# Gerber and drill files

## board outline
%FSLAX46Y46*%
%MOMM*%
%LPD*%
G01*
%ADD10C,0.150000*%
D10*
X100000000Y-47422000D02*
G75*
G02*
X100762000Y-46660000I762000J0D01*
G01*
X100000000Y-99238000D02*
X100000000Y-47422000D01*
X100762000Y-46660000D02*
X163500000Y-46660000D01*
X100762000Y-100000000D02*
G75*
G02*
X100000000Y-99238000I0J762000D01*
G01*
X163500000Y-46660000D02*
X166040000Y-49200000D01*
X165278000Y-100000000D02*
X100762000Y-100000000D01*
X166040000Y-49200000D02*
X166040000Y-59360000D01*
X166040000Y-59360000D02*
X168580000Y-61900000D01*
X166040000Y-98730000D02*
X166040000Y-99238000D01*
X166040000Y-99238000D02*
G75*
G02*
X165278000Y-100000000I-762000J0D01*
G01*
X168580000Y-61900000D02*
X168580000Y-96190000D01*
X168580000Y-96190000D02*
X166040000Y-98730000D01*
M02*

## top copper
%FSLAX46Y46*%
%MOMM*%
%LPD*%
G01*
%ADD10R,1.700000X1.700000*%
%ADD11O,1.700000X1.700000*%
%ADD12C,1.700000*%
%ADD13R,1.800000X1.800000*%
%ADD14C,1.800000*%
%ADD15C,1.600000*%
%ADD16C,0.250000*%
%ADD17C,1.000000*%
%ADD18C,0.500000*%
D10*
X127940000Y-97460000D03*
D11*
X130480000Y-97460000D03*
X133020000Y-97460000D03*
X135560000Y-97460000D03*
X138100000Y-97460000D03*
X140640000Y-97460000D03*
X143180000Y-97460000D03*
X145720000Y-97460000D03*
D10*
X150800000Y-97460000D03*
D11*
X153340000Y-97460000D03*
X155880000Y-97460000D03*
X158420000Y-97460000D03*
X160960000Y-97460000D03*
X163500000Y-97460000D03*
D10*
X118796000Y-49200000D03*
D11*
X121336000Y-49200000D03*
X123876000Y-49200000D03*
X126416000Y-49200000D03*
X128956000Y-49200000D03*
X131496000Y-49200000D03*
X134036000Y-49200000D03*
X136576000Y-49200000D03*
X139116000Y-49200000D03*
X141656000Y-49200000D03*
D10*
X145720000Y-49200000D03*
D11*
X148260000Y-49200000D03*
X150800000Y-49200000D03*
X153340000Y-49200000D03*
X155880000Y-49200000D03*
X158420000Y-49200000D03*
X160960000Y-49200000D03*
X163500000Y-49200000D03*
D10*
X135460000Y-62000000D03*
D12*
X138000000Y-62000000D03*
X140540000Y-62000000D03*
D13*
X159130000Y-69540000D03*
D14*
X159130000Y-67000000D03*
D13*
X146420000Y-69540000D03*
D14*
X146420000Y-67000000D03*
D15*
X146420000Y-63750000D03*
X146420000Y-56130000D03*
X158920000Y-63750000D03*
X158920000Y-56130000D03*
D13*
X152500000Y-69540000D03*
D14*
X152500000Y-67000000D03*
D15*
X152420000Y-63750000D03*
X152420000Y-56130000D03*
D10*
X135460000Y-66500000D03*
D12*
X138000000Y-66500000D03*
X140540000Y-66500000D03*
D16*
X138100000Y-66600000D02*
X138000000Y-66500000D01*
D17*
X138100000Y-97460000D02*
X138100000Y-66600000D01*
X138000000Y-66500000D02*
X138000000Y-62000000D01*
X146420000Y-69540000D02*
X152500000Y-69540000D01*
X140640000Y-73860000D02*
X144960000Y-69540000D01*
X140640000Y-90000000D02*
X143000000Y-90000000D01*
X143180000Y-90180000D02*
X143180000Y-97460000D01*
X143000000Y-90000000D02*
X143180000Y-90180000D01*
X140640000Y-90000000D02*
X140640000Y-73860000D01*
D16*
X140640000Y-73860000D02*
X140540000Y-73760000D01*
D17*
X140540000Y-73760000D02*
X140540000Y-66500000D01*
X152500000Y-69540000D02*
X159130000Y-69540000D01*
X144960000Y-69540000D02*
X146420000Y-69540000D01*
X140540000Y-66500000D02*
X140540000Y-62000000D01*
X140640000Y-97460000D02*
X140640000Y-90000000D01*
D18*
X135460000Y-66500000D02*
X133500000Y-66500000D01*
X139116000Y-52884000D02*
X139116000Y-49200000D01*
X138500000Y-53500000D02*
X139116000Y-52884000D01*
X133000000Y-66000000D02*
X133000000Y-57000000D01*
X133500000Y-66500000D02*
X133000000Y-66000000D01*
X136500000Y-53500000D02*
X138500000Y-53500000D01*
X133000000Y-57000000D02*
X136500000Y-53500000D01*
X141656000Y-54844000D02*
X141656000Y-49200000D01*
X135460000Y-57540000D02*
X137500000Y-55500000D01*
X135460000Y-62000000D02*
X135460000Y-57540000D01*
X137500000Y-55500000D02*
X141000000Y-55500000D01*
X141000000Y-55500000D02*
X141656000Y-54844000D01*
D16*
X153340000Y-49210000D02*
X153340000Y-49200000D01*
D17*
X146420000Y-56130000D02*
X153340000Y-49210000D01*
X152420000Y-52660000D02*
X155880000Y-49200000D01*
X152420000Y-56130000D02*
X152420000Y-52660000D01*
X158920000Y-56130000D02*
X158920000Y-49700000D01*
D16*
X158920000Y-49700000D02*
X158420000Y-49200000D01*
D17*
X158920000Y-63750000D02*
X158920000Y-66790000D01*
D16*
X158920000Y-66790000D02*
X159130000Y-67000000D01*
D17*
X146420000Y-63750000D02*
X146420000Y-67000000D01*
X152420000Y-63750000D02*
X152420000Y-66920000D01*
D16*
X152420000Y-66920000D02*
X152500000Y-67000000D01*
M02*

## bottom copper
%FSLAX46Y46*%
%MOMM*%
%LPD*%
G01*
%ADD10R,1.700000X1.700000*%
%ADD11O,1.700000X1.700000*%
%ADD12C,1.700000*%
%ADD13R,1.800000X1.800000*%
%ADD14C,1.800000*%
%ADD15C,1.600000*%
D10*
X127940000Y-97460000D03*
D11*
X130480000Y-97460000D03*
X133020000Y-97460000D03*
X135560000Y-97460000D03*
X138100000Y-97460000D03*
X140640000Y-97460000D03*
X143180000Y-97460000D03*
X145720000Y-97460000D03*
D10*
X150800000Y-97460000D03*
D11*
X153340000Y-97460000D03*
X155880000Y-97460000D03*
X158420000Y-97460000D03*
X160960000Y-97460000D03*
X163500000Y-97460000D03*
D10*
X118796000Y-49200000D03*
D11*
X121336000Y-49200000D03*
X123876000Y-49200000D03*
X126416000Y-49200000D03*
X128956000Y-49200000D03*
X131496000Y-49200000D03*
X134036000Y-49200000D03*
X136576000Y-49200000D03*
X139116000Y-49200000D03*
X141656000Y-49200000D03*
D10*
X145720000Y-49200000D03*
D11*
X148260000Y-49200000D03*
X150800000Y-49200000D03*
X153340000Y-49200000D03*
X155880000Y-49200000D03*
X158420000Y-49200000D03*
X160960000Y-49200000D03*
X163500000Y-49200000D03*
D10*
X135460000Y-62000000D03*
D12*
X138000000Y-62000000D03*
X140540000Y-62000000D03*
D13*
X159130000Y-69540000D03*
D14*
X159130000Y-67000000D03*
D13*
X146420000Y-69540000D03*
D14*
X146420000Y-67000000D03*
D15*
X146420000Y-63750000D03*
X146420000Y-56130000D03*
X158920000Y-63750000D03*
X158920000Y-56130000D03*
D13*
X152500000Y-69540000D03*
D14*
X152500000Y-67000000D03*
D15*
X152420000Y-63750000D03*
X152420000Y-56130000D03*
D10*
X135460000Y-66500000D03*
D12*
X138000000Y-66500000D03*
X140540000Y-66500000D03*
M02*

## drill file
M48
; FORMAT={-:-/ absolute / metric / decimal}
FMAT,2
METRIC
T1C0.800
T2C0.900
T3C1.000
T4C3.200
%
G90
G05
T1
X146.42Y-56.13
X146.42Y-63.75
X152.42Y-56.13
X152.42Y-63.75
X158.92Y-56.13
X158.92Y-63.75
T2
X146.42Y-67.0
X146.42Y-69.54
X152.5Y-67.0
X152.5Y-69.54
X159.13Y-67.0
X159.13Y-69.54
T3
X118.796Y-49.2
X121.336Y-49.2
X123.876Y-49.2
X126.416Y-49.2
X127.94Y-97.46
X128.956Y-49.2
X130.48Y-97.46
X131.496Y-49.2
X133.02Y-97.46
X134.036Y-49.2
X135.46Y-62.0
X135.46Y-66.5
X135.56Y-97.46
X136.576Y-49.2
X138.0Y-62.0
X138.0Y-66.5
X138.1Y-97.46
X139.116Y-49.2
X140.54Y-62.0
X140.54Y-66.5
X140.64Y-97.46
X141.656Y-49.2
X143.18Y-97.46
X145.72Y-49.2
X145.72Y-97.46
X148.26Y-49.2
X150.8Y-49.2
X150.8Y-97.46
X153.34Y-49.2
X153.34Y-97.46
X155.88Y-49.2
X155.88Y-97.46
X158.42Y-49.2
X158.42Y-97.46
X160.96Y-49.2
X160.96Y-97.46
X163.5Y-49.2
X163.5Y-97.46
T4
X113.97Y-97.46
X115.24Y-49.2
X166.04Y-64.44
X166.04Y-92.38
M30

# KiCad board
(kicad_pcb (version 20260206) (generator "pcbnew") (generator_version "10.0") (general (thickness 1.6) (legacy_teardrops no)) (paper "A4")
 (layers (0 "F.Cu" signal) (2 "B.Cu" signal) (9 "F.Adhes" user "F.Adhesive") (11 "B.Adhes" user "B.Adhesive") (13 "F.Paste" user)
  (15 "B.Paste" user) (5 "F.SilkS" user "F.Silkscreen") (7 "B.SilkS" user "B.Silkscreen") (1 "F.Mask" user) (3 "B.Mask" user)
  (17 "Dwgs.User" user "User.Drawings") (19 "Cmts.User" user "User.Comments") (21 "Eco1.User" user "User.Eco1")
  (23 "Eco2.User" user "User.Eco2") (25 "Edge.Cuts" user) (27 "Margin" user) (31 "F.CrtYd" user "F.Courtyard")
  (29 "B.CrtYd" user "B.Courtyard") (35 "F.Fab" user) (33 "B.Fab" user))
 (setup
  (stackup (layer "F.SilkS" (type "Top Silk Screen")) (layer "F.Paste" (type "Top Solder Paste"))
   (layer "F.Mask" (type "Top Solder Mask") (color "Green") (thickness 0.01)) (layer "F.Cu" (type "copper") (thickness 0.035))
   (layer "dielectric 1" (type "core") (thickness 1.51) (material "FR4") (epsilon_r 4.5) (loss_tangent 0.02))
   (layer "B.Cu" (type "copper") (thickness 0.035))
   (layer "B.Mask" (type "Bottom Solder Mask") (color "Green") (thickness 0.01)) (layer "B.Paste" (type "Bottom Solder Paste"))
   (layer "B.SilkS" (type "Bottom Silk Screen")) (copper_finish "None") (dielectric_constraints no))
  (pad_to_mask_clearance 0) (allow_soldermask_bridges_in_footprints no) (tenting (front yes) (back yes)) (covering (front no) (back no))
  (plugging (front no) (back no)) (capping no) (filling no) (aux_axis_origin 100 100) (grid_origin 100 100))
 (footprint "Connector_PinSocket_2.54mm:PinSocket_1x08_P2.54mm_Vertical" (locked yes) (layer "F.Cu") (at 127.94 97.46 90)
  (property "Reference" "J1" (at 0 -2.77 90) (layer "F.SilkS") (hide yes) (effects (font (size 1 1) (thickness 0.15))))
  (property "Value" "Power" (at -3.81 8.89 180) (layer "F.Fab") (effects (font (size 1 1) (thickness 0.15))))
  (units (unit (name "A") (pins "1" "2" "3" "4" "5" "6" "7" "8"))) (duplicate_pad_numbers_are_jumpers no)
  (pad "1" thru_hole rect (at 0 0 90) (size 1.7 1.7) (drill 1) (layers "*.Cu" "*.Mask") (remove_unused_layers no)
   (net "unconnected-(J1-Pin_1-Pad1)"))
  (pad "2" thru_hole oval (at 0 2.54 90) (size 1.7 1.7) (drill 1) (layers "*.Cu" "*.Mask") (remove_unused_layers no)
   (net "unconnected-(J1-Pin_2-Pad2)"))
  (pad "3" thru_hole oval (at 0 5.08 90) (size 1.7 1.7) (drill 1) (layers "*.Cu" "*.Mask") (remove_unused_layers no)
   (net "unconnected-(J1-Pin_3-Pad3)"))
  (pad "4" thru_hole oval (at 0 7.62 90) (size 1.7 1.7) (drill 1) (layers "*.Cu" "*.Mask") (remove_unused_layers no) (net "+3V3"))
  (pad "5" thru_hole oval (at 0 10.16 90) (size 1.7 1.7) (drill 1) (layers "*.Cu" "*.Mask") (remove_unused_layers no) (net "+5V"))
  (pad "6" thru_hole oval (at 0 12.7 90) (size 1.7 1.7) (drill 1) (layers "*.Cu" "*.Mask") (remove_unused_layers no) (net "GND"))
  (pad "7" thru_hole oval (at 0 15.24 90) (size 1.7 1.7) (drill 1) (layers "*.Cu" "*.Mask") (remove_unused_layers no) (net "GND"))
  (pad "8" thru_hole oval (at 0 17.78 90) (size 1.7 1.7) (drill 1) (layers "*.Cu" "*.Mask") (remove_unused_layers no)
   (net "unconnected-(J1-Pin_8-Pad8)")))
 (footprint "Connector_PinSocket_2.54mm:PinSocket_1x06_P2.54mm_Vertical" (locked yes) (layer "F.Cu") (at 150.8 97.46 90)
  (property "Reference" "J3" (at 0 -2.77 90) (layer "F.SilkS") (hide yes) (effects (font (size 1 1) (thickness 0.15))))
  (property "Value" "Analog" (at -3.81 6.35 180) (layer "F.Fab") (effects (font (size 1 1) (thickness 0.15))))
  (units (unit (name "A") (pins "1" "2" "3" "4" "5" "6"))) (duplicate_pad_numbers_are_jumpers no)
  (pad "1" thru_hole rect (at 0 0 90) (size 1.7 1.7) (drill 1) (layers "*.Cu" "*.Mask") (remove_unused_layers no) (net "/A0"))
  (pad "2" thru_hole oval (at 0 2.54 90) (size 1.7 1.7) (drill 1) (layers "*.Cu" "*.Mask") (remove_unused_layers no) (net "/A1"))
  (pad "3" thru_hole oval (at 0 5.08 90) (size 1.7 1.7) (drill 1) (layers "*.Cu" "*.Mask") (remove_unused_layers no) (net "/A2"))
  (pad "4" thru_hole oval (at 0 7.62 90) (size 1.7 1.7) (drill 1) (layers "*.Cu" "*.Mask") (remove_unused_layers no) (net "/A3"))
  (pad "5" thru_hole oval (at 0 10.16 90) (size 1.7 1.7) (drill 1) (layers "*.Cu" "*.Mask") (remove_unused_layers no)
   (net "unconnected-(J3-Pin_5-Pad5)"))
  (pad "6" thru_hole oval (at 0 12.7 90) (size 1.7 1.7) (drill 1) (layers "*.Cu" "*.Mask") (remove_unused_layers no)
   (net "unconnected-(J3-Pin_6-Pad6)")))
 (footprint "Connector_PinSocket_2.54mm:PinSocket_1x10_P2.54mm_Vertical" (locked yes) (layer "F.Cu") (at 118.796 49.2 90)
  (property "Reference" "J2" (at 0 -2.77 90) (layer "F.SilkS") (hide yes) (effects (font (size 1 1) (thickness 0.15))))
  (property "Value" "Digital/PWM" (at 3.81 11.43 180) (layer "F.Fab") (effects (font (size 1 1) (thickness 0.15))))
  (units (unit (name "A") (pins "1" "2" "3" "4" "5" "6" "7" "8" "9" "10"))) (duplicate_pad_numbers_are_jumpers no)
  (pad "1" thru_hole rect (at 0 0 90) (size 1.7 1.7) (drill 1) (layers "*.Cu" "*.Mask") (remove_unused_layers no) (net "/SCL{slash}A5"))
  (pad "2" thru_hole oval (at 0 2.54 90) (size 1.7 1.7) (drill 1) (layers "*.Cu" "*.Mask") (remove_unused_layers no) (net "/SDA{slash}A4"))
  (pad "3" thru_hole oval (at 0 5.08 90) (size 1.7 1.7) (drill 1) (layers "*.Cu" "*.Mask") (remove_unused_layers no) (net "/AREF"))
  (pad "4" thru_hole oval (at 0 7.62 90) (size 1.7 1.7) (drill 1) (layers "*.Cu" "*.Mask") (remove_unused_layers no)
   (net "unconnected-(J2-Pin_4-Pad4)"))
  (pad "5" thru_hole oval (at 0 10.16 90) (size 1.7 1.7) (drill 1) (layers "*.Cu" "*.Mask") (remove_unused_layers no) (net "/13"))
  (pad "6" thru_hole oval (at 0 12.7 90) (size 1.7 1.7) (drill 1) (layers "*.Cu" "*.Mask") (remove_unused_layers no) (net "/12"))
  (pad "7" thru_hole oval (at 0 15.24 90) (size 1.7 1.7) (drill 1) (layers "*.Cu" "*.Mask") (remove_unused_layers no) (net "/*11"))
  (pad "8" thru_hole oval (at 0 17.78 90) (size 1.7 1.7) (drill 1) (layers "*.Cu" "*.Mask") (remove_unused_layers no) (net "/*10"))
  (pad "9" thru_hole oval (at 0 20.32 90) (size 1.7 1.7) (drill 1) (layers "*.Cu" "*.Mask") (remove_unused_layers no) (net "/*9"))
  (pad "10" thru_hole oval (at 0 22.86 90) (size 1.7 1.7) (drill 1) (layers "*.Cu" "*.Mask") (remove_unused_layers no) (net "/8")))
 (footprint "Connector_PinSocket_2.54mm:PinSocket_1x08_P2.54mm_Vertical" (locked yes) (layer "F.Cu") (at 145.72 49.2 90)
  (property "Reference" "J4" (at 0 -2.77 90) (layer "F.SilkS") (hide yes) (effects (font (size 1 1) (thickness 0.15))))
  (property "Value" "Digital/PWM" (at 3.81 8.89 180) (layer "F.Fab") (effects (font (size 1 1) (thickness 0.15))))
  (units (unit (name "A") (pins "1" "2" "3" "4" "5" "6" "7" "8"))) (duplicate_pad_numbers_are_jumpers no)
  (pad "1" thru_hole rect (at 0 0 90) (size 1.7 1.7) (drill 1) (layers "*.Cu" "*.Mask") (remove_unused_layers no) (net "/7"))
  (pad "2" thru_hole oval (at 0 2.54 90) (size 1.7 1.7) (drill 1) (layers "*.Cu" "*.Mask") (remove_unused_layers no) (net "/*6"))
  (pad "3" thru_hole oval (at 0 5.08 90) (size 1.7 1.7) (drill 1) (layers "*.Cu" "*.Mask") (remove_unused_layers no) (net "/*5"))
  (pad "4" thru_hole oval (at 0 7.62 90) (size 1.7 1.7) (drill 1) (layers "*.Cu" "*.Mask") (remove_unused_layers no) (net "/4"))
  (pad "5" thru_hole oval (at 0 10.16 90) (size 1.7 1.7) (drill 1) (layers "*.Cu" "*.Mask") (remove_unused_layers no) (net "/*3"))
  (pad "6" thru_hole oval (at 0 12.7 90) (size 1.7 1.7) (drill 1) (layers "*.Cu" "*.Mask") (remove_unused_layers no) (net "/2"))
  (pad "7" thru_hole oval (at 0 15.24 90) (size 1.7 1.7) (drill 1) (layers "*.Cu" "*.Mask") (remove_unused_layers no) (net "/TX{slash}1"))
  (pad "8" thru_hole oval (at 0 17.78 90) (size 1.7 1.7) (drill 1) (layers "*.Cu" "*.Mask") (remove_unused_layers no) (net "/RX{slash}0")))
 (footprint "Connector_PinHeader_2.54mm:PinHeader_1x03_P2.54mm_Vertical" (layer "F.Cu") (at 135.46 62 90)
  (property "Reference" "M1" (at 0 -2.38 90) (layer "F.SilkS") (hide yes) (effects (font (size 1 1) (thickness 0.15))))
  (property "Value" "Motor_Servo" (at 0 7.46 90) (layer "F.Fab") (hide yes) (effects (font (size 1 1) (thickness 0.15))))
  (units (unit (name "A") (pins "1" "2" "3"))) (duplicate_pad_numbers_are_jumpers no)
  (pad "1" thru_hole rect (at 0 0 90) (size 1.7 1.7) (drill 1) (layers "*.Cu" "*.Mask") (remove_unused_layers no) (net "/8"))
  (pad "2" thru_hole circle (at 0 2.54 90) (size 1.7 1.7) (drill 1) (layers "*.Cu" "*.Mask") (remove_unused_layers no) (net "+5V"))
  (pad "3" thru_hole circle (at 0 5.08 90) (size 1.7 1.7) (drill 1) (layers "*.Cu" "*.Mask") (remove_unused_layers no) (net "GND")))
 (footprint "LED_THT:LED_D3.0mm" (layer "F.Cu") (at 159.13 69.54 90)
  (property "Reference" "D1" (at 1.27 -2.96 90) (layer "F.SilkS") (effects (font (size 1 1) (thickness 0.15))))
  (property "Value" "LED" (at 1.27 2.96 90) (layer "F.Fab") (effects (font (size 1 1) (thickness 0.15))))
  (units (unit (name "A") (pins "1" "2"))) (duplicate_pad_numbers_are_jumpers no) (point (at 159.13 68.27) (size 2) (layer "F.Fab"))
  (pad "1" thru_hole rect (at 0 0 90) (size 1.8 1.8) (drill 0.9) (layers "*.Cu" "*.Mask") (remove_unused_layers no) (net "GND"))
  (pad "2" thru_hole circle (at 2.54 0 90) (size 1.8 1.8) (drill 0.9) (layers "*.Cu" "*.Mask") (remove_unused_layers no) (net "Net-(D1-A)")))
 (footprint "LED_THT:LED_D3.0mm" (layer "F.Cu") (at 146.42 69.54 90)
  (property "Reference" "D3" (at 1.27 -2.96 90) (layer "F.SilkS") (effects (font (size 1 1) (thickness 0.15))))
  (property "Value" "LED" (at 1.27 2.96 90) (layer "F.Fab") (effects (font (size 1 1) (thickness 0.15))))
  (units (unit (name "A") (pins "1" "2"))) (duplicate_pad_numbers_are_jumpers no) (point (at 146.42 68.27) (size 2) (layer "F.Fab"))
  (pad "1" thru_hole rect (at 0 0 90) (size 1.8 1.8) (drill 0.9) (layers "*.Cu" "*.Mask") (remove_unused_layers no) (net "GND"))
  (pad "2" thru_hole circle (at 2.54 0 90) (size 1.8 1.8) (drill 0.9) (layers "*.Cu" "*.Mask") (remove_unused_layers no) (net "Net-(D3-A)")))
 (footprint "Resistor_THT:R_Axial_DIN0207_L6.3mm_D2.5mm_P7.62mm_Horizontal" (layer "F.Cu") (at 146.42 63.75 90)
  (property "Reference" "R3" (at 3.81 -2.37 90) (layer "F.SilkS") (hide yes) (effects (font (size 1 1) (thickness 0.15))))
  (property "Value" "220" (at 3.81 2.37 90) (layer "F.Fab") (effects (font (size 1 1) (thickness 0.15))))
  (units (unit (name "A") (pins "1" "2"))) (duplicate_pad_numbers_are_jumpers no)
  (pad "1" thru_hole circle (at 0 0 90) (size 1.6 1.6) (drill 0.8) (layers "*.Cu" "*.Mask") (remove_unused_layers no) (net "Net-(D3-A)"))
  (pad "2" thru_hole circle (at 7.62 0 90) (size 1.6 1.6) (drill 0.8) (layers "*.Cu" "*.Mask") (remove_unused_layers no) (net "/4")))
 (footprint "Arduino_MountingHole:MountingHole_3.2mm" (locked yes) (layer "F.Cu") (at 115.24 49.2)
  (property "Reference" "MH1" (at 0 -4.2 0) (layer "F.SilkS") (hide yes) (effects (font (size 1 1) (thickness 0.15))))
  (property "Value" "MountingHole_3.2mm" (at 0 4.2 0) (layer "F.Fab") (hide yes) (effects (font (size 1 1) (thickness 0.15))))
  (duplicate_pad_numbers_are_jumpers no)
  (pad "" np_thru_hole circle (at 0 0) (size 3.2 3.2) (drill 3.2) (layers "*.Cu" "*.Mask")))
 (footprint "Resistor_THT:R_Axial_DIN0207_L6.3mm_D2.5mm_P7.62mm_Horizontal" (layer "F.Cu") (at 158.92 63.75 90)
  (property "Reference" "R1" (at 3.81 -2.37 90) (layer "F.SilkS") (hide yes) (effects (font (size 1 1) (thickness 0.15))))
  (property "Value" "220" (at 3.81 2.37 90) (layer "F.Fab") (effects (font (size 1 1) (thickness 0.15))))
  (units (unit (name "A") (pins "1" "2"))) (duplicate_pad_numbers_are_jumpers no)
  (pad "1" thru_hole circle (at 0 0 90) (size 1.6 1.6) (drill 0.8) (layers "*.Cu" "*.Mask") (remove_unused_layers no) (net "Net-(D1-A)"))
  (pad "2" thru_hole circle (at 7.62 0 90) (size 1.6 1.6) (drill 0.8) (layers "*.Cu" "*.Mask") (remove_unused_layers no) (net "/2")))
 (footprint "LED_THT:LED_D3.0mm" (layer "F.Cu") (at 152.5 69.54 90)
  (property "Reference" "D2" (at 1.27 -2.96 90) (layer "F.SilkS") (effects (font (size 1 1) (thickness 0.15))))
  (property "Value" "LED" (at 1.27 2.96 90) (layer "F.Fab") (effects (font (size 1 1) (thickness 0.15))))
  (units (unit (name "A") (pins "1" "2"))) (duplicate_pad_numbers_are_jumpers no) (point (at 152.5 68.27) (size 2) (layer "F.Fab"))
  (pad "1" thru_hole rect (at 0 0 90) (size 1.8 1.8) (drill 0.9) (layers "*.Cu" "*.Mask") (remove_unused_layers no) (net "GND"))
  (pad "2" thru_hole circle (at 2.54 0 90) (size 1.8 1.8) (drill 0.9) (layers "*.Cu" "*.Mask") (remove_unused_layers no) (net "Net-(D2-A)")))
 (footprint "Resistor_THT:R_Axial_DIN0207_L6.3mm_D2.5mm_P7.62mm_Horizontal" (layer "F.Cu") (at 152.42 63.75 90)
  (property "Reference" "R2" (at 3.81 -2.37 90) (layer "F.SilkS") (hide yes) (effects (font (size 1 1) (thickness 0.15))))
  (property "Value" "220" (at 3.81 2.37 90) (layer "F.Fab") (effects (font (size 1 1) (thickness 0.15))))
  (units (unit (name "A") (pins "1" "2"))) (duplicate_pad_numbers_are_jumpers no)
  (pad "1" thru_hole circle (at 0 0 90) (size 1.6 1.6) (drill 0.8) (layers "*.Cu" "*.Mask") (remove_unused_layers no) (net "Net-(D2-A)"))
  (pad "2" thru_hole circle (at 7.62 0 90) (size 1.6 1.6) (drill 0.8) (layers "*.Cu" "*.Mask") (remove_unused_layers no) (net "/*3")))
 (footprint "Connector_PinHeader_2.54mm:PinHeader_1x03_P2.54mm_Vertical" (layer "F.Cu") (at 135.46 66.5 90)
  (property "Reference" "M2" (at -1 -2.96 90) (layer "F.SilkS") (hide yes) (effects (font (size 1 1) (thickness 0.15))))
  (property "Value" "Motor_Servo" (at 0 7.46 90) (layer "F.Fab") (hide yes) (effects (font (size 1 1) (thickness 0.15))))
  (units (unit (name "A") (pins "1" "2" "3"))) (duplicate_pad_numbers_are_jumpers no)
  (pad "1" thru_hole rect (at 0 0 90) (size 1.7 1.7) (drill 1) (layers "*.Cu" "*.Mask") (remove_unused_layers no) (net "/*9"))
  (pad "2" thru_hole circle (at 0 2.54 90) (size 1.7 1.7) (drill 1) (layers "*.Cu" "*.Mask") (remove_unused_layers no) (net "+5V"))
  (pad "3" thru_hole circle (at 0 5.08 90) (size 1.7 1.7) (drill 1) (layers "*.Cu" "*.Mask") (remove_unused_layers no) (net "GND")))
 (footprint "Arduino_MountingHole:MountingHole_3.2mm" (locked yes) (layer "F.Cu") (at 113.97 97.46)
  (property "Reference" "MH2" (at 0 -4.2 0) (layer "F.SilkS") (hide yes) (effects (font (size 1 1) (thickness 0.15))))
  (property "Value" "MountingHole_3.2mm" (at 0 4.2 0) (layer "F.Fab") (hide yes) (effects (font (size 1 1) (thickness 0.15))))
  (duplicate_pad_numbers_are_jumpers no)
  (pad "" np_thru_hole circle (at 0 0) (size 3.2 3.2) (drill 3.2) (layers "*.Cu" "*.Mask")))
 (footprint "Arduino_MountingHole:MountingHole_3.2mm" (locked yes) (layer "F.Cu") (at 166.04 64.44)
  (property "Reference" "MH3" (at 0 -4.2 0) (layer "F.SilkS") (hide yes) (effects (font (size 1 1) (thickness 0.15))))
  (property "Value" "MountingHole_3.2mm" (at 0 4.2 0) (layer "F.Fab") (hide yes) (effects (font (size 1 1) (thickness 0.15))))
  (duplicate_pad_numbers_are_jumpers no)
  (pad "" np_thru_hole circle (at 0 0) (size 3.2 3.2) (drill 3.2) (layers "*.Cu" "*.Mask")))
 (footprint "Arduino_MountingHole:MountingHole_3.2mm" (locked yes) (layer "F.Cu") (at 166.04 92.38)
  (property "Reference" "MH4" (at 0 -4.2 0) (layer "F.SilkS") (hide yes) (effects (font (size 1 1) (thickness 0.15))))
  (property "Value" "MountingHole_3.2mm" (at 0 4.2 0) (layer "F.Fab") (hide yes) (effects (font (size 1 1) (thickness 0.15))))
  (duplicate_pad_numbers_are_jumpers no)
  (pad "" np_thru_hole circle (at 0 0) (size 3.2 3.2) (drill 3.2) (layers "*.Cu" "*.Mask")))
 (gr_arc (start 100 47.422) (mid 100.223185 46.883185) (end 100.762 46.66) (stroke (width 0.15) (type solid)) (layer "Edge.Cuts"))
 (gr_line (start 100 99.238) (end 100 47.422) (stroke (width 0.15) (type solid)) (layer "Edge.Cuts"))
 (gr_line (start 100.762 46.66) (end 163.5 46.66) (stroke (width 0.15) (type solid)) (layer "Edge.Cuts"))
 (gr_arc (start 100.762 100) (mid 100.223185 99.776815) (end 100 99.238) (stroke (width 0.15) (type solid)) (layer "Edge.Cuts"))
 (gr_line (start 163.5 46.66) (end 166.04 49.2) (stroke (width 0.15) (type solid)) (layer "Edge.Cuts"))
 (gr_line (start 165.278 100) (end 100.762 100) (stroke (width 0.15) (type solid)) (layer "Edge.Cuts"))
 (gr_line (start 166.04 49.2) (end 166.04 59.36) (stroke (width 0.15) (type solid)) (layer "Edge.Cuts"))
 (gr_line (start 166.04 59.36) (end 168.58 61.9) (stroke (width 0.15) (type solid)) (layer "Edge.Cuts"))
 (gr_line (start 166.04 98.73) (end 166.04 99.238) (stroke (width 0.15) (type solid)) (layer "Edge.Cuts"))
 (gr_arc (start 166.04 99.238) (mid 165.816815 99.776815) (end 165.278 100) (stroke (width 0.15) (type solid)) (layer "Edge.Cuts"))
 (gr_line (start 168.58 61.9) (end 168.58 96.19) (stroke (width 0.15) (type solid)) (layer "Edge.Cuts"))
 (gr_line (start 168.58 96.19) (end 166.04 98.73) (stroke (width 0.15) (type solid)) (layer "Edge.Cuts"))
 (segment (start 138.1 66.6) (end 138 66.5) (width 0.25) (layer "F.Cu") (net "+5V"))
 (segment (start 138.1 97.46) (end 138.1 66.6) (width 1) (layer "F.Cu") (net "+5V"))
 (segment (start 138 66.5) (end 138 62) (width 1) (layer "F.Cu") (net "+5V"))
 (segment (start 146.42 69.54) (end 152.5 69.54) (width 1) (layer "F.Cu") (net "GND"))
 (segment (start 140.64 73.86) (end 144.96 69.54) (width 1) (layer "F.Cu") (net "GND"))
 (segment (start 140.64 90) (end 143 90) (width 1) (layer "F.Cu") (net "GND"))
 (segment (start 143.18 90.18) (end 143.18 97.46) (width 1) (layer "F.Cu") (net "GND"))
 (segment (start 143 90) (end 143.18 90.18) (width 1) (layer "F.Cu") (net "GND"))
 (segment (start 140.64 90) (end 140.64 73.86) (width 1) (layer "F.Cu") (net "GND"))
 (segment (start 140.64 73.86) (end 140.54 73.76) (width 0.25) (layer "F.Cu") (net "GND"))
 (segment (start 140.54 73.76) (end 140.54 66.5) (width 1) (layer "F.Cu") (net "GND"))
 (segment (start 152.5 69.54) (end 159.13 69.54) (width 1) (layer "F.Cu") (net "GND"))
 (segment (start 144.96 69.54) (end 146.42 69.54) (width 1) (layer "F.Cu") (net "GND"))
 (segment (start 140.54 66.5) (end 140.54 62) (width 1) (layer "F.Cu") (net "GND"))
 (segment (start 140.64 97.46) (end 140.64 90) (width 1) (layer "F.Cu") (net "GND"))
 (segment (start 135.46 66.5) (end 133.5 66.5) (width 0.5) (layer "F.Cu") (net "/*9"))
 (segment (start 139.116 52.884) (end 139.116 49.2) (width 0.5) (layer "F.Cu") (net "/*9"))
 (segment (start 138.5 53.5) (end 139.116 52.884) (width 0.5) (layer "F.Cu") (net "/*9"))
 (segment (start 133 66) (end 133 57) (width 0.5) (layer "F.Cu") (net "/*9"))
 (segment (start 133.5 66.5) (end 133 66) (width 0.5) (layer "F.Cu") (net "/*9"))
 (segment (start 136.5 53.5) (end 138.5 53.5) (width 0.5) (layer "F.Cu") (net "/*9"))
 (segment (start 133 57) (end 136.5 53.5) (width 0.5) (layer "F.Cu") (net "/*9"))
 (segment (start 141.656 54.844) (end 141.656 49.2) (width 0.5) (layer "F.Cu") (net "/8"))
 (segment (start 135.46 57.54) (end 137.5 55.5) (width 0.5) (layer "F.Cu") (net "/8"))
 (segment (start 135.46 62) (end 135.46 57.54) (width 0.5) (layer "F.Cu") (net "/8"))
 (segment (start 137.5 55.5) (end 141 55.5) (width 0.5) (layer "F.Cu") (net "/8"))
 (segment (start 141 55.5) (end 141.656 54.844) (width 0.5) (layer "F.Cu") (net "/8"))
 (segment (start 153.34 49.21) (end 153.34 49.2) (width 0.25) (layer "F.Cu") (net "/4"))
 (segment (start 146.42 56.13) (end 153.34 49.21) (width 1) (layer "F.Cu") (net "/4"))
 (segment (start 152.42 52.66) (end 155.88 49.2) (width 1) (layer "F.Cu") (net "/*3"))
 (segment (start 152.42 56.13) (end 152.42 52.66) (width 1) (layer "F.Cu") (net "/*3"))
 (segment (start 158.92 56.13) (end 158.92 49.7) (width 1) (layer "F.Cu") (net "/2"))
 (segment (start 158.92 49.7) (end 158.42 49.2) (width 0.25) (layer "F.Cu") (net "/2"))
 (segment (start 158.92 63.75) (end 158.92 66.79) (width 1) (layer "F.Cu") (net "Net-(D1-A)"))
 (segment (start 158.92 66.79) (end 159.13 67) (width 0.25) (layer "F.Cu") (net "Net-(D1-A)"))
 (segment (start 146.42 63.75) (end 146.42 67) (width 1) (layer "F.Cu") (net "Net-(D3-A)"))
 (segment (start 152.42 63.75) (end 152.42 66.92) (width 1) (layer "F.Cu") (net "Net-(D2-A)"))
 (segment (start 152.42 66.92) (end 152.5 67) (width 0.25) (layer "F.Cu") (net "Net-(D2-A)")))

